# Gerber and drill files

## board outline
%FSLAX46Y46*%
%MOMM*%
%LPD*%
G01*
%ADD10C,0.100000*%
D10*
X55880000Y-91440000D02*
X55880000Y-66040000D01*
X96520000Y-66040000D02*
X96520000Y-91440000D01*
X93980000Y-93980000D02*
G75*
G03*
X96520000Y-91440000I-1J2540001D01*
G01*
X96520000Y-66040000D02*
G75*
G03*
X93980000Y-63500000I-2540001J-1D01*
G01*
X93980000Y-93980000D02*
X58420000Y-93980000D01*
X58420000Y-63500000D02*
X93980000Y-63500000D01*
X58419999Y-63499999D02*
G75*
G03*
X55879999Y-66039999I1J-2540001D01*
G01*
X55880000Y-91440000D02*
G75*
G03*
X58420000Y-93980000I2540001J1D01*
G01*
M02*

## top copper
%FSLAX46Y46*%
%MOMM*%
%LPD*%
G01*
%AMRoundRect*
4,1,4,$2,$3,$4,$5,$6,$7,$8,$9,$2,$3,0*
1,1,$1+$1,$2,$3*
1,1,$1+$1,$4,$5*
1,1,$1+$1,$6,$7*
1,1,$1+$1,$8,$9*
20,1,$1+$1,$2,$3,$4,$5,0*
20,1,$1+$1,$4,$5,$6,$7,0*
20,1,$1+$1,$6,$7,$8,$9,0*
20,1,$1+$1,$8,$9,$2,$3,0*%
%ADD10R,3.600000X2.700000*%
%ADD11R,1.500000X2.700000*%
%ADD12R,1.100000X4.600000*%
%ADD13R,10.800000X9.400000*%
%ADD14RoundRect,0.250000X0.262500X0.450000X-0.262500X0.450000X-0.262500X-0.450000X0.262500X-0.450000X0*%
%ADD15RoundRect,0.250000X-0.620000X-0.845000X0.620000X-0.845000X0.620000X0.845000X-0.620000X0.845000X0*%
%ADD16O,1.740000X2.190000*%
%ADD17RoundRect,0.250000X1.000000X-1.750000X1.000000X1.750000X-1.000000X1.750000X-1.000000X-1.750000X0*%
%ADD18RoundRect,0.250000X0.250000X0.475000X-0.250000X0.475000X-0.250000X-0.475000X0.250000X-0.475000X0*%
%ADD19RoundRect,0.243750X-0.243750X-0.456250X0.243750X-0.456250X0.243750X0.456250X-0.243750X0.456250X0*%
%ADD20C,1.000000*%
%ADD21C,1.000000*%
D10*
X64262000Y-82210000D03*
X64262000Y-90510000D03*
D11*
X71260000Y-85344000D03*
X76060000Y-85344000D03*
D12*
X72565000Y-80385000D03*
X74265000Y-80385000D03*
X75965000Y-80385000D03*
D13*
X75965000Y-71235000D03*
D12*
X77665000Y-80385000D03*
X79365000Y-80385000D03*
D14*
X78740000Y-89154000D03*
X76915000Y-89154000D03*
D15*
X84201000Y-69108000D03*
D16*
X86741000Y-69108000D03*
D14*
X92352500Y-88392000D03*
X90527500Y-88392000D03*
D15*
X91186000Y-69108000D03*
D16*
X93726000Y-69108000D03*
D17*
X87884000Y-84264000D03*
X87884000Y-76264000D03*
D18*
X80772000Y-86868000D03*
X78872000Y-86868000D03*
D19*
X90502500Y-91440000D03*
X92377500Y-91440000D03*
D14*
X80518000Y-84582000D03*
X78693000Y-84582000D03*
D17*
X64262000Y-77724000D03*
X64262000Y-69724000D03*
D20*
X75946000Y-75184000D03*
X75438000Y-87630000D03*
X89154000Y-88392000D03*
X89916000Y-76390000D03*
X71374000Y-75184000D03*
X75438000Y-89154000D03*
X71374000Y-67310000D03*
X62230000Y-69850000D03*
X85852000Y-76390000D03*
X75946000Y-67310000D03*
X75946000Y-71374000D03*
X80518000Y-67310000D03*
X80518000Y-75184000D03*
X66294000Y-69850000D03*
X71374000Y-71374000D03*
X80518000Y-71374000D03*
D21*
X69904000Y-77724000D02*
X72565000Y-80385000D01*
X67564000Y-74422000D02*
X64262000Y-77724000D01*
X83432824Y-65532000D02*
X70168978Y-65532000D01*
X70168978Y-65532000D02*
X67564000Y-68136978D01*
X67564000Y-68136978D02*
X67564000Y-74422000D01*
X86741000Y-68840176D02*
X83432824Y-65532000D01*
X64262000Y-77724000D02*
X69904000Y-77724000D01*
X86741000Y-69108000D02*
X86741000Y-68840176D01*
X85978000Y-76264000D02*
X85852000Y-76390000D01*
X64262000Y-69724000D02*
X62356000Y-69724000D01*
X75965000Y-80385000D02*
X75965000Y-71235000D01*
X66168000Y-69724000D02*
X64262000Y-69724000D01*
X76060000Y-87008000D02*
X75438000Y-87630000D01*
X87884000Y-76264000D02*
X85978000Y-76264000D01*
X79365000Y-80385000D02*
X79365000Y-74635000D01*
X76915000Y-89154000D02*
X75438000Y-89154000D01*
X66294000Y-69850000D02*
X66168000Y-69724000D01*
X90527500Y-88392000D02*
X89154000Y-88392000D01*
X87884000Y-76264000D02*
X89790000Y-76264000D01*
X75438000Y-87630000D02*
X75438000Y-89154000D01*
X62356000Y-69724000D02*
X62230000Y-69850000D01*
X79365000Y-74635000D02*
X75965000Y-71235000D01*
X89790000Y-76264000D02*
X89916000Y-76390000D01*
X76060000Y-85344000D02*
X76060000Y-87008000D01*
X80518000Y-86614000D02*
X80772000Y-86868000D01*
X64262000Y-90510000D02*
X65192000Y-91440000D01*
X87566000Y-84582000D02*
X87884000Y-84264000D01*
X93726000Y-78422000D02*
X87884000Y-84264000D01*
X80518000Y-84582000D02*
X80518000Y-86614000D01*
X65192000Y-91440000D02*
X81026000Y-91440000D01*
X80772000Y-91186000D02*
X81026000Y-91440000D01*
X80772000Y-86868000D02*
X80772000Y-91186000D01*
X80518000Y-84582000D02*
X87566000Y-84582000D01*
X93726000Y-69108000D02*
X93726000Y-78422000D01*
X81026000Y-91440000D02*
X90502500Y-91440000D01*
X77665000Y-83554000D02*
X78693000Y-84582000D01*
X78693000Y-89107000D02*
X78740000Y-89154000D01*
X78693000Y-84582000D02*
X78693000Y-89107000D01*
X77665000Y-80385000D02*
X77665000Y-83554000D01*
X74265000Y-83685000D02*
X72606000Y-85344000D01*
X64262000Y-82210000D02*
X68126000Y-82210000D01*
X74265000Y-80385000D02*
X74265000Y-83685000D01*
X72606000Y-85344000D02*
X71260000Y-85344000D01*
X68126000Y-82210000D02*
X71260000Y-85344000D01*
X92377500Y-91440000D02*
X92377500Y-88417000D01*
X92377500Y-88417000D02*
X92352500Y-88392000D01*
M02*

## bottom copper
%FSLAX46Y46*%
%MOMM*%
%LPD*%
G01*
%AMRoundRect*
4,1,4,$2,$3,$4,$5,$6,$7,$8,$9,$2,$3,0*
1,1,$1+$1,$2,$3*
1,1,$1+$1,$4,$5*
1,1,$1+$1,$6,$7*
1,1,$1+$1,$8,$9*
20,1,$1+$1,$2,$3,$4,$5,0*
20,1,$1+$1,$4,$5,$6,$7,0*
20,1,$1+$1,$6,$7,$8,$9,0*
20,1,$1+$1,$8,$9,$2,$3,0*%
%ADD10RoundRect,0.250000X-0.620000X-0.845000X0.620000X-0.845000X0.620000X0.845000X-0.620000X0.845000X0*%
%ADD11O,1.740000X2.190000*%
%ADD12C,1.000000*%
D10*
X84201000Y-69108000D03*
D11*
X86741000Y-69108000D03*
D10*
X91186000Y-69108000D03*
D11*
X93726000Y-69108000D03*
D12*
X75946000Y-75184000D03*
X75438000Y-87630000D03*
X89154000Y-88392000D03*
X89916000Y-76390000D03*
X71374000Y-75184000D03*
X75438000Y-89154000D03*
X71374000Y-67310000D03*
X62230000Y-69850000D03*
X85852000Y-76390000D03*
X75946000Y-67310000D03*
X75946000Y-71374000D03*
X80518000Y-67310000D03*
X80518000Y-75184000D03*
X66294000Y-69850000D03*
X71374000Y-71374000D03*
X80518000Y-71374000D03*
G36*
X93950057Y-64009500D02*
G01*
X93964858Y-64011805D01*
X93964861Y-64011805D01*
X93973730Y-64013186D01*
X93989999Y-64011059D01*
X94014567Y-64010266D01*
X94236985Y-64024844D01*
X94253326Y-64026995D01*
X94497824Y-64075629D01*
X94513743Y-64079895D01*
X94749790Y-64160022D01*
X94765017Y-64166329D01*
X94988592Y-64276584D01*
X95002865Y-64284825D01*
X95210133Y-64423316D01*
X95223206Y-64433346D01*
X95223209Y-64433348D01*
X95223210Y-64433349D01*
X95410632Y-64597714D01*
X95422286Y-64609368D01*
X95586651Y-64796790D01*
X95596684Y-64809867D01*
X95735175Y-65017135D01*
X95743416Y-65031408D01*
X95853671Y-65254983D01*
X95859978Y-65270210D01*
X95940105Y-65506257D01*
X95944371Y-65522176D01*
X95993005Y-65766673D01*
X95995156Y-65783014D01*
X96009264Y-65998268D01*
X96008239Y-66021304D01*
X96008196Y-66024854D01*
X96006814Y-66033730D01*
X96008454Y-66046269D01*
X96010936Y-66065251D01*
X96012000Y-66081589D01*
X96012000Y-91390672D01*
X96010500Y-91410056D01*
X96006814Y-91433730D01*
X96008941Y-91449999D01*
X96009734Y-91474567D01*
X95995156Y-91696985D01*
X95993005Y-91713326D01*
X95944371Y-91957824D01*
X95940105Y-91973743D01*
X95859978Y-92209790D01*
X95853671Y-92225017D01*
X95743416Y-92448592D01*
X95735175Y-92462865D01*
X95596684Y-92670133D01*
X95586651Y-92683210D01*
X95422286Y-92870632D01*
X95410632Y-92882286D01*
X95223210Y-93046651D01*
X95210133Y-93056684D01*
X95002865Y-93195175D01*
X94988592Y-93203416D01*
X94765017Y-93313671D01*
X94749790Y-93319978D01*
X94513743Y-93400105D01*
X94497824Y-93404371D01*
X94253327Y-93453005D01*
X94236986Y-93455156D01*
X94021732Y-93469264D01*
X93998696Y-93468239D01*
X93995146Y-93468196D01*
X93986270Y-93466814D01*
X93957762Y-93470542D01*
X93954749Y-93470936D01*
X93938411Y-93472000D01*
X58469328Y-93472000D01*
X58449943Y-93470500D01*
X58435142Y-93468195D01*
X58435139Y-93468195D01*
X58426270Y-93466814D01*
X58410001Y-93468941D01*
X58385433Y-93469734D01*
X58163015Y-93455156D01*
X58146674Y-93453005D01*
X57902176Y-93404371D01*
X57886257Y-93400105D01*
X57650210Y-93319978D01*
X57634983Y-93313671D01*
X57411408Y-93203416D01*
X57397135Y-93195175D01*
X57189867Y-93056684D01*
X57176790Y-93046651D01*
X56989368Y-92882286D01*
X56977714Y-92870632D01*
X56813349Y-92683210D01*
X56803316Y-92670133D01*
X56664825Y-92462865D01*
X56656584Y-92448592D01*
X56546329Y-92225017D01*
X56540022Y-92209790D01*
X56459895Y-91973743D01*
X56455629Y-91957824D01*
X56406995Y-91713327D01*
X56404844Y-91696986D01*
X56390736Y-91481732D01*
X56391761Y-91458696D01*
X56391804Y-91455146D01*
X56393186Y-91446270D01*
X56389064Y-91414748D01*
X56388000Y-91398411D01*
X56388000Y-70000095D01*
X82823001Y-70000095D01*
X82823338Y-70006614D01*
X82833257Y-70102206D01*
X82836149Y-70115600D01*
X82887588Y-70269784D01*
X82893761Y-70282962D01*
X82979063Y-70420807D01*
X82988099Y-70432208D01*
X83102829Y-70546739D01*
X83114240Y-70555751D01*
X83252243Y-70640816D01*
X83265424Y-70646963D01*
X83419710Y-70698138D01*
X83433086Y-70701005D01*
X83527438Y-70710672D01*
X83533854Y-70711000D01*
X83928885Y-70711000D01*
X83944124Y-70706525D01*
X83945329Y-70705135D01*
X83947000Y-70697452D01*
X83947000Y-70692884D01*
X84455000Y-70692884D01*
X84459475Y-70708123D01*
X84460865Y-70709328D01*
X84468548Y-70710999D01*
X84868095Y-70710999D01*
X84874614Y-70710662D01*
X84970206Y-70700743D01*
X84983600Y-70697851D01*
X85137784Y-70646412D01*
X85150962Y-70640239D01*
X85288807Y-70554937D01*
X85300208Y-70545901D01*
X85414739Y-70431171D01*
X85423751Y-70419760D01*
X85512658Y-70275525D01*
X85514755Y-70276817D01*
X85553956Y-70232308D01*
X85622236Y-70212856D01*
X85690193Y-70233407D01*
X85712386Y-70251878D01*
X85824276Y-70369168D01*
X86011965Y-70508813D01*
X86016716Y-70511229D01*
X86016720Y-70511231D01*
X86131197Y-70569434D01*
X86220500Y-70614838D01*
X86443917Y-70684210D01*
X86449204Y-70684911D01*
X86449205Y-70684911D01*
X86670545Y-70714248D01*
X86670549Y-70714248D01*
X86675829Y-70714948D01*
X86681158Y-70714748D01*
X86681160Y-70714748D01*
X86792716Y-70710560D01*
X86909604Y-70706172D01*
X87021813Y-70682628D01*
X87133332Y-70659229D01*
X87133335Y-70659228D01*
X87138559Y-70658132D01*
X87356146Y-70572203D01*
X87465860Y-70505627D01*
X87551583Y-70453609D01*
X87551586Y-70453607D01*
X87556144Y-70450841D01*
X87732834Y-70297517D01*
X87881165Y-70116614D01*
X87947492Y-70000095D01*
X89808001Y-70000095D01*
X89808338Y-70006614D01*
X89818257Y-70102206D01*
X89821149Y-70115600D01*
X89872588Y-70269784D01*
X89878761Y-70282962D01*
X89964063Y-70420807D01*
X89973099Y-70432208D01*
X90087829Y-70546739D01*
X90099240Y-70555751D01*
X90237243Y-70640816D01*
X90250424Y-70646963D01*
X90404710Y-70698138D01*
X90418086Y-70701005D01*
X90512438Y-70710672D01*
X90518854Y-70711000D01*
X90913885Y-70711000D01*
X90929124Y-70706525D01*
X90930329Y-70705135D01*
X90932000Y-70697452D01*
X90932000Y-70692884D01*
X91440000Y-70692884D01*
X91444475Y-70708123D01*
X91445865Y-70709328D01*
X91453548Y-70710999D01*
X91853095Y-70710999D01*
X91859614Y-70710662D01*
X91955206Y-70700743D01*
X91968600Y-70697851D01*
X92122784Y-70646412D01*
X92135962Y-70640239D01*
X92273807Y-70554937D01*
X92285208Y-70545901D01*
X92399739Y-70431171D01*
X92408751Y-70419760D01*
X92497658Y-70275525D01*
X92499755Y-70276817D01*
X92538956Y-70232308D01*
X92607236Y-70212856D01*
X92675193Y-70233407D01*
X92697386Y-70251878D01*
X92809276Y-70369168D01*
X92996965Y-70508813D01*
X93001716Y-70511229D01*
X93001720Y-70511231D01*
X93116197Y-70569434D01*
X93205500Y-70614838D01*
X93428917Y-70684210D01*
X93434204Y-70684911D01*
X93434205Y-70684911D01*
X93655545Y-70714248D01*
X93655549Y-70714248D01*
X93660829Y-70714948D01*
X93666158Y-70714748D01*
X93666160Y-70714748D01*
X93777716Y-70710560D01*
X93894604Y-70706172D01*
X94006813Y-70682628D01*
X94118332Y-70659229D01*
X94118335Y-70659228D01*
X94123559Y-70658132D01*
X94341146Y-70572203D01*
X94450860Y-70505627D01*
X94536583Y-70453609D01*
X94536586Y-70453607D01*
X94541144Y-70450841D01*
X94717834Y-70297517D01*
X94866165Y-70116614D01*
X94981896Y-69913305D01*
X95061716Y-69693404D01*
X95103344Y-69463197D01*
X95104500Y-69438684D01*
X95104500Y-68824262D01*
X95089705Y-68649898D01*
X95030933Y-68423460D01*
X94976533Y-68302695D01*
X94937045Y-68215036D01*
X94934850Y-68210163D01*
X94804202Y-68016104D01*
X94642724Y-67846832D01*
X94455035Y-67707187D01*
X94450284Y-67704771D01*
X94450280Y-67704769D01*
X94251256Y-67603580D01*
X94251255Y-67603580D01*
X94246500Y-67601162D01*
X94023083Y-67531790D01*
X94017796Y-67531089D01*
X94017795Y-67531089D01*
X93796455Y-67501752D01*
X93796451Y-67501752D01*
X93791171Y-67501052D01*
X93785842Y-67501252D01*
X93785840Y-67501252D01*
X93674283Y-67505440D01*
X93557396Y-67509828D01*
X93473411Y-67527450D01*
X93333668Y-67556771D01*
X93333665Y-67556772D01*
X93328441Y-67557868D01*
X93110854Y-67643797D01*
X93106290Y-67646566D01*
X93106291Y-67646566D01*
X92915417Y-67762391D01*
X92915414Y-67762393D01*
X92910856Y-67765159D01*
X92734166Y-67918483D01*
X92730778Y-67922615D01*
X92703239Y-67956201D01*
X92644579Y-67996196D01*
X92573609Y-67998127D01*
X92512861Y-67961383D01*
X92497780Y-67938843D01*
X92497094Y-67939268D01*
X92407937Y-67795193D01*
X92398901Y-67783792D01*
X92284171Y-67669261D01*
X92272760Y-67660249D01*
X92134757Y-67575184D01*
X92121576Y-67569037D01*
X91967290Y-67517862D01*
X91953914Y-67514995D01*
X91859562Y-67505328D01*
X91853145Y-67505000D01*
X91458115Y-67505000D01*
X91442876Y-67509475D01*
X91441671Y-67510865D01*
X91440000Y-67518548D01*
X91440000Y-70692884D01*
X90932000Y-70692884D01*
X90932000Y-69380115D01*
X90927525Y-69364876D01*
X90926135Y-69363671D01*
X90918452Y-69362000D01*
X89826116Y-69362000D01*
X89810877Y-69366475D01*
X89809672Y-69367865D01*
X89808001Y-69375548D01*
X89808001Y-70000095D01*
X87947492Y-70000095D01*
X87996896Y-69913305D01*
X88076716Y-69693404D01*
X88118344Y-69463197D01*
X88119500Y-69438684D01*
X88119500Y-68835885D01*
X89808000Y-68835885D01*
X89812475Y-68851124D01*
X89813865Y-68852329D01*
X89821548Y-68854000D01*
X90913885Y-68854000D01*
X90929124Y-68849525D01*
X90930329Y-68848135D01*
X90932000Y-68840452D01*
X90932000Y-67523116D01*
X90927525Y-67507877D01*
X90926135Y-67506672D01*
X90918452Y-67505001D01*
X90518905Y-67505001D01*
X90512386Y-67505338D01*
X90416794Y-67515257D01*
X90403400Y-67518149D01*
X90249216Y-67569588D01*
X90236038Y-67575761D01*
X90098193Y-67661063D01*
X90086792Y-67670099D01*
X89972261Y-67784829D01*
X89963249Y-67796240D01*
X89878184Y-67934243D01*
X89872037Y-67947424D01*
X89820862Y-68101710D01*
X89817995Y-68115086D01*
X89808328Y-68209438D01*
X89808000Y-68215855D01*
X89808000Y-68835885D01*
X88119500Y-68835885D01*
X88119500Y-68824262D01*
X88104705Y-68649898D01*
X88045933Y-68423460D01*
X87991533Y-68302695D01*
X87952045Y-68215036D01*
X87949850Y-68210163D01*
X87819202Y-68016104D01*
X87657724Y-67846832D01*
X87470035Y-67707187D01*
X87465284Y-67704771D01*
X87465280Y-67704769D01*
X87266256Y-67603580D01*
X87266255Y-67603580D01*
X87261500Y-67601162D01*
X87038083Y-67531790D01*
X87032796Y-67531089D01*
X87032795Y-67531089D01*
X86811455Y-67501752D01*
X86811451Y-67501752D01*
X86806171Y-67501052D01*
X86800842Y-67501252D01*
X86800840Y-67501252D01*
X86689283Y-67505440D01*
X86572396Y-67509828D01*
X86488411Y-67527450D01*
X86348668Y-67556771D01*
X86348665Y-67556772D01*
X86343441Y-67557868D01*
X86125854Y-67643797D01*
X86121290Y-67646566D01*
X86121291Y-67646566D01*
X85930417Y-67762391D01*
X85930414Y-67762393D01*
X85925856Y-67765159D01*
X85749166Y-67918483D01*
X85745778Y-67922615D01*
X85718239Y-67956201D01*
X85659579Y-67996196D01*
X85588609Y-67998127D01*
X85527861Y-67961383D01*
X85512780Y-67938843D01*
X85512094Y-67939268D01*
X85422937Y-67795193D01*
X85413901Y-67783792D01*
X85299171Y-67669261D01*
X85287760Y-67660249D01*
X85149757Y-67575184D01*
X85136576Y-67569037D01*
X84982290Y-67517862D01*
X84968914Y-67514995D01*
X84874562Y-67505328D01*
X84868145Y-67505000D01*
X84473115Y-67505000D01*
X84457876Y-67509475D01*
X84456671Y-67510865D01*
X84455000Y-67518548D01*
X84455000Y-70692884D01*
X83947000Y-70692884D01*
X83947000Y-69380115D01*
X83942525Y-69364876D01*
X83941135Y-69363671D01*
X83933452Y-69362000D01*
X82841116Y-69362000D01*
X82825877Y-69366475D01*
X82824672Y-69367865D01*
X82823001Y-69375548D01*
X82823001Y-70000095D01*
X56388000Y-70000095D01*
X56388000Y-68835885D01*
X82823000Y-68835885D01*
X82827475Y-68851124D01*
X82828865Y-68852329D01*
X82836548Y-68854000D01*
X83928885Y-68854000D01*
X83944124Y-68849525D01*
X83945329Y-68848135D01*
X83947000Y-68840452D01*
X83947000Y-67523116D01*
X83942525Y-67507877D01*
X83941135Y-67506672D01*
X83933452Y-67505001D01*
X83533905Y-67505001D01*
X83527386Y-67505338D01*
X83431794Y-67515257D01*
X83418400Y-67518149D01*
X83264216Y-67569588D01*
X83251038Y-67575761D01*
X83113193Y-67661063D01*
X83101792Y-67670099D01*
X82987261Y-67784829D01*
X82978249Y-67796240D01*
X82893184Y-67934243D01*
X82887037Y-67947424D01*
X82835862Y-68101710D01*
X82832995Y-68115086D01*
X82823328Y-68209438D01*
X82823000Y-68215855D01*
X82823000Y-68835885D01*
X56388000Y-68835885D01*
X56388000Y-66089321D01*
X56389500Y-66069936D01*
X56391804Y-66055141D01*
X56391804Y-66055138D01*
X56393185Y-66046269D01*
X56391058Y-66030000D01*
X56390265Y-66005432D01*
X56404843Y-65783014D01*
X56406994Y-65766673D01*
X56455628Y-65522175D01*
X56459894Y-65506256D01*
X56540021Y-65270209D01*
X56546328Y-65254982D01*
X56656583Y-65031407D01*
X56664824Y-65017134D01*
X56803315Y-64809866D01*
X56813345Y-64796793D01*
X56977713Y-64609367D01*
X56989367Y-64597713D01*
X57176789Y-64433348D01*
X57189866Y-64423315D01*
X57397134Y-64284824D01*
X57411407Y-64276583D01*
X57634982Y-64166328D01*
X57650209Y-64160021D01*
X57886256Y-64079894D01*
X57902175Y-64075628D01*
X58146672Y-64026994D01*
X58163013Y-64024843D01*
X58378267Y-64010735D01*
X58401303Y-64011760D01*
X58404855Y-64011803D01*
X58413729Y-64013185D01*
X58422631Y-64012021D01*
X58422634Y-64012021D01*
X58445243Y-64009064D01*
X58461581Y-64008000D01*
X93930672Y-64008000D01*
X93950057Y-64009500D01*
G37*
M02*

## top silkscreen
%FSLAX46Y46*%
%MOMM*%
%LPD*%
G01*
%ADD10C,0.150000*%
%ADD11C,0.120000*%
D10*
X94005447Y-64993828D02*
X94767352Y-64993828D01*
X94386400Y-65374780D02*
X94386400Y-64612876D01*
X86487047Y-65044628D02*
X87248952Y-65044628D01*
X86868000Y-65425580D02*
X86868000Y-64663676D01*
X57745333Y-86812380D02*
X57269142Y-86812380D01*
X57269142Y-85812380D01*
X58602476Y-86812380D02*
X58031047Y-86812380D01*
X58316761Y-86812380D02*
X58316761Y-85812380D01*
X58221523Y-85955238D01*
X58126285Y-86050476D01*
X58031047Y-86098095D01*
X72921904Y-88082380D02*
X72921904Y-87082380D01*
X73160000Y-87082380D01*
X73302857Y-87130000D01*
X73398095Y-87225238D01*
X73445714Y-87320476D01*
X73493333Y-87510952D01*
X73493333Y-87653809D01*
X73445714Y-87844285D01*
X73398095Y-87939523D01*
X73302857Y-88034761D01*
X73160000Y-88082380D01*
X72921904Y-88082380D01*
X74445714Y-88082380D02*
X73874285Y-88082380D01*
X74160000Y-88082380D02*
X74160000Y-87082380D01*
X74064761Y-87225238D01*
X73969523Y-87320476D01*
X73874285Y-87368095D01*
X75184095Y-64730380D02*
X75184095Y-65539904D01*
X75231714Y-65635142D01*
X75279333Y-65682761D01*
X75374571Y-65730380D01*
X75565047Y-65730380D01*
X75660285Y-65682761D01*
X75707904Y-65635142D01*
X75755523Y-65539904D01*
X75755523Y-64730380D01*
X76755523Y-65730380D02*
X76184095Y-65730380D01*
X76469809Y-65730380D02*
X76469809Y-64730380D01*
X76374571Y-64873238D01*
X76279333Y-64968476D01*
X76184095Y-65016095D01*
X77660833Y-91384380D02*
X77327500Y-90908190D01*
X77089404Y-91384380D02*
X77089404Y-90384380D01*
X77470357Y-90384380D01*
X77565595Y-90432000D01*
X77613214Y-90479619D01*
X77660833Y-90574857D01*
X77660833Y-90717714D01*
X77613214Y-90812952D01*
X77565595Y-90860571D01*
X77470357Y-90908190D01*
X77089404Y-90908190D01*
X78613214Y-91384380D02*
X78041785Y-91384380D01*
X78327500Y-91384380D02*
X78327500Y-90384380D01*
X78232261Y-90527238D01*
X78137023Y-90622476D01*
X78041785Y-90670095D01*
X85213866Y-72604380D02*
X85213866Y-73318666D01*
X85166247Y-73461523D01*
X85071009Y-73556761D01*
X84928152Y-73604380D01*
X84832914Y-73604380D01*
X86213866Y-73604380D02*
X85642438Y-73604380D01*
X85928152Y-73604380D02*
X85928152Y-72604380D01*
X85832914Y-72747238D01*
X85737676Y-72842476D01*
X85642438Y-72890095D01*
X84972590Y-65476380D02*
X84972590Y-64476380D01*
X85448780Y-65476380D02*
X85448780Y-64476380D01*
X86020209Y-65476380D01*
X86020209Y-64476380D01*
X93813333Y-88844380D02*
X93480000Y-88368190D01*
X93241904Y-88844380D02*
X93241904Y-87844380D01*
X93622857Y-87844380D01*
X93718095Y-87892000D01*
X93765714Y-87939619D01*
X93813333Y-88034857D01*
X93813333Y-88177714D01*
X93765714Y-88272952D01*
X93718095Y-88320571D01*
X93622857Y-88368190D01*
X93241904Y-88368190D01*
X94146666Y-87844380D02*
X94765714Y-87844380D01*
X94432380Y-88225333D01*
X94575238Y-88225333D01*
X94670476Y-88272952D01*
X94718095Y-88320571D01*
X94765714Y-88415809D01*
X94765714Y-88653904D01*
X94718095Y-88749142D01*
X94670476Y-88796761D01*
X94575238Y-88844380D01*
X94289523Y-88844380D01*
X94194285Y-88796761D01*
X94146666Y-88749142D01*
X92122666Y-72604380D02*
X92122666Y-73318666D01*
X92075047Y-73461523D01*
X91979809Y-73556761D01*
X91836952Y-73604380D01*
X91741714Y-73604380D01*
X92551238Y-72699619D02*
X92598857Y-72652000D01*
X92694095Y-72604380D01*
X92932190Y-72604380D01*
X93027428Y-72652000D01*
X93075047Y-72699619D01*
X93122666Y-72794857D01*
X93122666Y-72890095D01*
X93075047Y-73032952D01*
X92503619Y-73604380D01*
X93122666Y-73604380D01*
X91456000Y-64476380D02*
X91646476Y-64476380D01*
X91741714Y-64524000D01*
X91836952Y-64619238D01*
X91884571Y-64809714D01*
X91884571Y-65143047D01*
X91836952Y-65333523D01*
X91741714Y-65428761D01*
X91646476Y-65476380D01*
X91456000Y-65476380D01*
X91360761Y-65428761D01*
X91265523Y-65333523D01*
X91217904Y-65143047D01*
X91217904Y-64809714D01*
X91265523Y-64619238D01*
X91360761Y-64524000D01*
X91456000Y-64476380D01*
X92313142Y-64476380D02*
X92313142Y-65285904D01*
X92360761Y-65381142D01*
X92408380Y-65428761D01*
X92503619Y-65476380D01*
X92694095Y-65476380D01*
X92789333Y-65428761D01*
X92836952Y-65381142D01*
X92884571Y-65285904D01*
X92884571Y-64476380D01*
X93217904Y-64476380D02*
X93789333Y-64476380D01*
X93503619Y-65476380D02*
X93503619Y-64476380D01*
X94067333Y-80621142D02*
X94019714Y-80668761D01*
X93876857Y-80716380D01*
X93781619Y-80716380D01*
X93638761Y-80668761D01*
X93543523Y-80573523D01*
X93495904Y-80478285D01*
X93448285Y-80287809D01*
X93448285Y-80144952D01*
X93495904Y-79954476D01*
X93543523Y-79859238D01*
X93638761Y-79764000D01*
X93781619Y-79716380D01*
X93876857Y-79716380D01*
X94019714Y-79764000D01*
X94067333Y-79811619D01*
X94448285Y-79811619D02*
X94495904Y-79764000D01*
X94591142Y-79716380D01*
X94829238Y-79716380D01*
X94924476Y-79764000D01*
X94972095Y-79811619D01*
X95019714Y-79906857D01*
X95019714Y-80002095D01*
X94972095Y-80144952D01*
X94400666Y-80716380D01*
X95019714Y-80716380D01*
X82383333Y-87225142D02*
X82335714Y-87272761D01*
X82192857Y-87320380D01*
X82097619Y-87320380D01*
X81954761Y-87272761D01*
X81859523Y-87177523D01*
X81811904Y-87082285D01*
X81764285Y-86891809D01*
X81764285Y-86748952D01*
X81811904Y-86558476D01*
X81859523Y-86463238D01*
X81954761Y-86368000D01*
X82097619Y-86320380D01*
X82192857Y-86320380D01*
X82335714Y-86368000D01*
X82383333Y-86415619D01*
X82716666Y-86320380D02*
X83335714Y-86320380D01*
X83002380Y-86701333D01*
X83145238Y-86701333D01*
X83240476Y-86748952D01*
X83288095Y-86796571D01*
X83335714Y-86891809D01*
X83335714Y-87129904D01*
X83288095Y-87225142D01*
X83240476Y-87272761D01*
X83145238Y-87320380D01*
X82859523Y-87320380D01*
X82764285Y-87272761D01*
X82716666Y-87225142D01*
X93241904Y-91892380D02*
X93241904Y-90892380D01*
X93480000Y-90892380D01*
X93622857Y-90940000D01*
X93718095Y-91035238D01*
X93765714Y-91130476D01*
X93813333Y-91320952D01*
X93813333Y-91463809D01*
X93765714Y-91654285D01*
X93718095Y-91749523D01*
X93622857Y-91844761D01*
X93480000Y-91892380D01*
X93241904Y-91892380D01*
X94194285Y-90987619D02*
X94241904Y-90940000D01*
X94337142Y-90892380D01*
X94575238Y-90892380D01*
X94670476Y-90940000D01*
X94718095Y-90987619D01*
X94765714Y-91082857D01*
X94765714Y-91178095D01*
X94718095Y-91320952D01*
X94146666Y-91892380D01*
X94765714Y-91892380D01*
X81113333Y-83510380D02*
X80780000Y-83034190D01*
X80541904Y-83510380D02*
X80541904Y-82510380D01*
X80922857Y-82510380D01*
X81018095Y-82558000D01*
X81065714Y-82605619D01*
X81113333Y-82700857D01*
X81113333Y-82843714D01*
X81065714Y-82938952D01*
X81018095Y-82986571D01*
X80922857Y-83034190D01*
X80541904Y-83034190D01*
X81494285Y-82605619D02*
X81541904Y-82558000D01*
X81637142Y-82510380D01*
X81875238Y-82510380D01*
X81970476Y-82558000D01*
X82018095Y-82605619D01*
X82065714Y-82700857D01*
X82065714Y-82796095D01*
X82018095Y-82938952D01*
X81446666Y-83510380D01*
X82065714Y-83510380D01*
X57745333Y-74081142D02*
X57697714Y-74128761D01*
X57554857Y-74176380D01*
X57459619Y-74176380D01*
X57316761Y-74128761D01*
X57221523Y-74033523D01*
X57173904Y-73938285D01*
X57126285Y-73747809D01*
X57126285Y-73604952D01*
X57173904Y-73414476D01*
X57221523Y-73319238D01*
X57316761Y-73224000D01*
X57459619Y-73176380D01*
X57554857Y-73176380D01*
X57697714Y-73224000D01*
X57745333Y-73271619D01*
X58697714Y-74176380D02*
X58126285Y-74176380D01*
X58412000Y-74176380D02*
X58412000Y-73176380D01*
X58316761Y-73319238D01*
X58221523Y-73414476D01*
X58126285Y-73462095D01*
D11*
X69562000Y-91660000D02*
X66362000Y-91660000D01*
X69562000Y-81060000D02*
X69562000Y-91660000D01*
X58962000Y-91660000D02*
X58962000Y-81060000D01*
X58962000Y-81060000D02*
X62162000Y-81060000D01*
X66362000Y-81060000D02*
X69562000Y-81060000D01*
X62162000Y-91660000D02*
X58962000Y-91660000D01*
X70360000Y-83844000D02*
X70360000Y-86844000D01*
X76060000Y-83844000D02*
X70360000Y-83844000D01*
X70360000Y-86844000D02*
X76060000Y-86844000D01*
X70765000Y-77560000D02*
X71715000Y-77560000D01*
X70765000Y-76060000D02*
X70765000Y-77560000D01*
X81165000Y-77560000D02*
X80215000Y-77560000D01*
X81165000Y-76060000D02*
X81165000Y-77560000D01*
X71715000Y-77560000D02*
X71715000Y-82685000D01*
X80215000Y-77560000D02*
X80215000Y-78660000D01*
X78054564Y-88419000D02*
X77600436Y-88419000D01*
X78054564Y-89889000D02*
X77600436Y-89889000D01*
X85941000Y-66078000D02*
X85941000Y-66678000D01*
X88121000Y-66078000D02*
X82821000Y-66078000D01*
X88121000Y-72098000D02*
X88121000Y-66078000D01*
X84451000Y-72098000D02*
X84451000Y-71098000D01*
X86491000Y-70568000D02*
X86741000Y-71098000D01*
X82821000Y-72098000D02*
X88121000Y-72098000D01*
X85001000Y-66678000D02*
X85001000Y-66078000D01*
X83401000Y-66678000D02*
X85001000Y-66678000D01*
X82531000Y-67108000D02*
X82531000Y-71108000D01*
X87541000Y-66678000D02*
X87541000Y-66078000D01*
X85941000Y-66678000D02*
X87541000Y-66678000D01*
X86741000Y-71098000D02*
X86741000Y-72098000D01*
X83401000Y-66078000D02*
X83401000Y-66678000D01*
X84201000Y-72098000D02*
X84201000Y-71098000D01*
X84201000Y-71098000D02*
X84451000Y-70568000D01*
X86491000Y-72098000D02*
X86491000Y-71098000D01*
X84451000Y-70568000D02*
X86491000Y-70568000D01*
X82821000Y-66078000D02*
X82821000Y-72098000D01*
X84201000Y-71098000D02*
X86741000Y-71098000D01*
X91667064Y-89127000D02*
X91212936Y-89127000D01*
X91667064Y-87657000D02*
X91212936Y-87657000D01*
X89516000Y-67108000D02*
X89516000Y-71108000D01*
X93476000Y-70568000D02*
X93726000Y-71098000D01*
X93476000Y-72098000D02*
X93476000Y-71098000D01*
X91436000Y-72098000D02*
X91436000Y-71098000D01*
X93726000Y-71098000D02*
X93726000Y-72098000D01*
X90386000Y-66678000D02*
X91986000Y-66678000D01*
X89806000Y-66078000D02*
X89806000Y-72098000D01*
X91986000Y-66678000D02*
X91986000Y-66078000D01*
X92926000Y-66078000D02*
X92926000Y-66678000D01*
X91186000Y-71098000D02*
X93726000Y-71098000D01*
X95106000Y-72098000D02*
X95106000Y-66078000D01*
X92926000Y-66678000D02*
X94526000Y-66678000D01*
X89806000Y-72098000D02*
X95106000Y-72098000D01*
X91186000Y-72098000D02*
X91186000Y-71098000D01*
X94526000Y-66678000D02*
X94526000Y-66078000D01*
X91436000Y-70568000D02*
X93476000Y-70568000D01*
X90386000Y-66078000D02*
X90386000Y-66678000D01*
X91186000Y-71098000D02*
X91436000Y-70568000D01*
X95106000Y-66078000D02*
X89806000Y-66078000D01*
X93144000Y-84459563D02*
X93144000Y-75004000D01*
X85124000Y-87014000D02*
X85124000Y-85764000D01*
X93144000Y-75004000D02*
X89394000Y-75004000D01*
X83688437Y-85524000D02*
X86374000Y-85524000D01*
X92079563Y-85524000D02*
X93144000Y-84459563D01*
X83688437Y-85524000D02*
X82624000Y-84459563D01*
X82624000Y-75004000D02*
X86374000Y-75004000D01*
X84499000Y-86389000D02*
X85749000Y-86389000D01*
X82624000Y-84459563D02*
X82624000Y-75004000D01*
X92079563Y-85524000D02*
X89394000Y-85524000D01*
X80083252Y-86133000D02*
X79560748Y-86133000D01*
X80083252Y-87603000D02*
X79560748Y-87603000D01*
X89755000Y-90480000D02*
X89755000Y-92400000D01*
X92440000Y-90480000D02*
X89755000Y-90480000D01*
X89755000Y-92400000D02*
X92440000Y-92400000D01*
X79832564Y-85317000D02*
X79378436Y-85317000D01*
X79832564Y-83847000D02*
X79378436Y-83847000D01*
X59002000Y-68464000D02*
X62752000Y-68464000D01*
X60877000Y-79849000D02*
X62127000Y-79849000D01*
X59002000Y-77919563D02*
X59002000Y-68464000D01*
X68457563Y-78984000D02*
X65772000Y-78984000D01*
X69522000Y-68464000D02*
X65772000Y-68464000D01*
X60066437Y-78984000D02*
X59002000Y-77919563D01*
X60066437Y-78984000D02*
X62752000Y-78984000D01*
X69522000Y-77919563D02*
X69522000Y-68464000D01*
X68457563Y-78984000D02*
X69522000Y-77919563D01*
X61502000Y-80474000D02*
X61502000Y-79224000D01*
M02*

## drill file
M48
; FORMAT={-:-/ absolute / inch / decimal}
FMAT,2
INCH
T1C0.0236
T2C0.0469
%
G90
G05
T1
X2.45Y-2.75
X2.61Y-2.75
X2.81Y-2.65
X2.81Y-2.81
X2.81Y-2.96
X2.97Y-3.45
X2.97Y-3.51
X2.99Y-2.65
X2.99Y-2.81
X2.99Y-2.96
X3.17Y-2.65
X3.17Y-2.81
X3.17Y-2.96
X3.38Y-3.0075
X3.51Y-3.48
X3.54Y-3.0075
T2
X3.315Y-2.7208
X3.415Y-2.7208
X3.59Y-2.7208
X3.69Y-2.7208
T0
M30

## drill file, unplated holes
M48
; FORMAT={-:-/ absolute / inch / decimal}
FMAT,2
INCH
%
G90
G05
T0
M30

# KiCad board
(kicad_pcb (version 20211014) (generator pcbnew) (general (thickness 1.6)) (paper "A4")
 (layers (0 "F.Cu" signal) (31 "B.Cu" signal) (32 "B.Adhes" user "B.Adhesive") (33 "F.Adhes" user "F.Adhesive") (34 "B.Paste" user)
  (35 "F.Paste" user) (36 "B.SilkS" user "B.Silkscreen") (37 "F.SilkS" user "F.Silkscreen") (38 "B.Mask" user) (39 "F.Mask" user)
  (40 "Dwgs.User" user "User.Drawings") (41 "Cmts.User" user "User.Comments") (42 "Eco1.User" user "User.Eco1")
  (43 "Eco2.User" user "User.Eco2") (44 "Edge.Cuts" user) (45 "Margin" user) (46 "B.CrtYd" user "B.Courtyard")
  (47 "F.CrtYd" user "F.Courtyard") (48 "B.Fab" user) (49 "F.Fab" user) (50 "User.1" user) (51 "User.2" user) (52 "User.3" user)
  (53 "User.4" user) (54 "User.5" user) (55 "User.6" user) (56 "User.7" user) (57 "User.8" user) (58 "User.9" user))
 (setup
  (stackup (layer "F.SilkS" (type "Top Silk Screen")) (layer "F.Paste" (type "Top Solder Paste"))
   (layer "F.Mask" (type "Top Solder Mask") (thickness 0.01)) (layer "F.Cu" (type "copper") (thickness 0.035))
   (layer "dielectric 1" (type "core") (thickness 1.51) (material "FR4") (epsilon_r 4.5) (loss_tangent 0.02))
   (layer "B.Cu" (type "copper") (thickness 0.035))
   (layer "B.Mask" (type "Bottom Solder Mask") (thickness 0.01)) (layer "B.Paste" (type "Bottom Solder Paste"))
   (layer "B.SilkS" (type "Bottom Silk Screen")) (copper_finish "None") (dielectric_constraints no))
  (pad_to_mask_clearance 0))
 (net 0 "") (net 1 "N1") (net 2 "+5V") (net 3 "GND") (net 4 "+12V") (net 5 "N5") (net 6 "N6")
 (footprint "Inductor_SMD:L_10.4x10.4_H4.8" (layer "F.Cu") (at 64.262 86.36 -90)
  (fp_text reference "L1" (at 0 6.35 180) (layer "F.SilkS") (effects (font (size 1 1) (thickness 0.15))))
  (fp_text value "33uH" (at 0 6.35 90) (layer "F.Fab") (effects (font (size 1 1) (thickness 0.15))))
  (fp_line (start 5.3 -5.3) (end 5.3 -2.1) (layer "F.SilkS") (width 0.12))
  (fp_line (start -5.3 -5.3) (end 5.3 -5.3) (layer "F.SilkS") (width 0.12))
  (fp_line (start 5.3 5.3) (end -5.3 5.3) (layer "F.SilkS") (width 0.12))
  (fp_line (start -5.3 5.3) (end -5.3 2.1) (layer "F.SilkS") (width 0.12))
  (fp_line (start -5.3 -2.1) (end -5.3 -5.3) (layer "F.SilkS") (width 0.12))
  (fp_line (start 5.3 2.1) (end 5.3 5.3) (layer "F.SilkS") (width 0.12))
  (pad "1" smd rect locked (at -4.15 0 270) (size 2.7 3.6) (layers "F.Cu" "F.Paste" "F.Mask") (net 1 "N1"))
  (pad "2" smd rect locked (at 4.15 0 270) (size 2.7 3.6) (layers "F.Cu" "F.Paste" "F.Mask") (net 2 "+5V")))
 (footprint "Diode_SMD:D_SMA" (layer "F.Cu") (at 73.66 85.344)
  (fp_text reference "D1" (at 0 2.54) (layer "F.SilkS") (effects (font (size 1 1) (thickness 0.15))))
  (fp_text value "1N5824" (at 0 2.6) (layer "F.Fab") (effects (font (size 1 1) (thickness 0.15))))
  (fp_line (start -3.4 -1.65) (end 2 -1.65) (layer "F.SilkS") (width 0.12))
  (fp_line (start -3.4 -1.65) (end -3.4 1.65) (layer "F.SilkS") (width 0.12))
  (fp_line (start -3.4 1.65) (end 2 1.65) (layer "F.SilkS") (width 0.12))
  (pad "1" smd rect locked (at -2 0) (size 2.5 1.8) (layers "F.Cu" "F.Paste" "F.Mask") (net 1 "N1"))
  (pad "2" smd rect locked (at 2 0) (size 2.5 1.8) (layers "F.Cu" "F.Paste" "F.Mask") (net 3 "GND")))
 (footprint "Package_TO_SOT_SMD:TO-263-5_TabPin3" (layer "F.Cu") (at 75.965 74.61 90)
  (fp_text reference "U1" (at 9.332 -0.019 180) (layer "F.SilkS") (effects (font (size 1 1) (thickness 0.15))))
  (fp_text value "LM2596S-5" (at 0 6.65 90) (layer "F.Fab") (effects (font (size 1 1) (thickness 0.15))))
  (fp_line (start -2.95 -5.2) (end -2.95 -4.25) (layer "F.SilkS") (width 0.12))
  (fp_line (start -1.45 -5.2) (end -2.95 -5.2) (layer "F.SilkS") (width 0.12))
  (fp_line (start -2.95 5.2) (end -2.95 4.25) (layer "F.SilkS") (width 0.12))
  (fp_line (start -1.45 5.2) (end -2.95 5.2) (layer "F.SilkS") (width 0.12))
  (fp_line (start -2.95 -4.25) (end -8.075 -4.25) (layer "F.SilkS") (width 0.12))
  (fp_line (start -2.95 4.25) (end -4.05 4.25) (layer "F.SilkS") (width 0.12))
  (pad "" smd rect locked (at 5.8 -2.775 90) (size 4.55 5.25) (layers "F.Paste"))
  (pad "" smd rect locked (at 5.8 2.775 90) (size 4.55 5.25) (layers "F.Paste"))
  (pad "" smd rect locked (at 0.95 2.775 90) (size 4.55 5.25) (layers "F.Paste"))
  (pad "" smd rect locked (at 0.95 -2.775 90) (size 4.55 5.25) (layers "F.Paste"))
  (pad "1" smd rect locked (at -5.775 -3.4 90) (size 4.6 1.1) (layers "F.Cu" "F.Paste" "F.Mask") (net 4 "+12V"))
  (pad "2" smd rect locked (at -5.775 -1.7 90) (size 4.6 1.1) (layers "F.Cu" "F.Paste" "F.Mask") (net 1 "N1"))
  (pad "3" smd rect locked (at -5.775 0 90) (size 4.6 1.1) (layers "F.Cu" "F.Paste" "F.Mask") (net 3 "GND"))
  (pad "3" smd rect locked (at 3.375 0 90) (size 9.4 10.8) (layers "F.Cu" "F.Mask") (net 3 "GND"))
  (pad "4" smd rect locked (at -5.775 1.7 90) (size 4.6 1.1) (layers "F.Cu" "F.Paste" "F.Mask") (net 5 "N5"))
  (pad "5" smd rect locked (at -5.775 3.4 90) (size 4.6 1.1) (layers "F.Cu" "F.Paste" "F.Mask") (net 3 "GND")))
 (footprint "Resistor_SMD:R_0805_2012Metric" (layer "F.Cu") (at 77.8275 89.154 180)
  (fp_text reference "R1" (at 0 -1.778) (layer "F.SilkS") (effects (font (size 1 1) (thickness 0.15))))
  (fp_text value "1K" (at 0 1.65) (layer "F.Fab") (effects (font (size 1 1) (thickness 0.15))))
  (fp_line (start -0.227064 0.735) (end 0.227064 0.735) (layer "F.SilkS") (width 0.12))
  (fp_line (start -0.227064 -0.735) (end 0.227064 -0.735) (layer "F.SilkS") (width 0.12))
  (pad "1" smd roundrect locked (at -0.9125 0 180) (size 1.025 1.4) (layers "F.Cu" "F.Paste" "F.Mask") (roundrect_rratio 0.243902439)
   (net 5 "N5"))
  (pad "2" smd roundrect locked (at 0.9125 0 180) (size 1.025 1.4) (layers "F.Cu" "F.Paste" "F.Mask") (roundrect_rratio 0.243902439)
   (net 3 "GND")))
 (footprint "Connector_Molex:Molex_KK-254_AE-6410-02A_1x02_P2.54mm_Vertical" (layer "F.Cu") (at 84.201 69.108)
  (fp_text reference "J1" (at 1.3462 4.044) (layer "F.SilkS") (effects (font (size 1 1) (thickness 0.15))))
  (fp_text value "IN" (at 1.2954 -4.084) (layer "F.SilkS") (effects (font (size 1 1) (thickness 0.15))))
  (fp_line (start 1.74 -3.03) (end 1.74 -2.43) (layer "F.SilkS") (width 0.12))
  (fp_line (start 3.92 -3.03) (end -1.38 -3.03) (layer "F.SilkS") (width 0.12))
  (fp_line (start 3.92 2.99) (end 3.92 -3.03) (layer "F.SilkS") (width 0.12))
  (fp_line (start 0.25 2.99) (end 0.25 1.99) (layer "F.SilkS") (width 0.12))
  (fp_line (start 2.29 1.46) (end 2.54 1.99) (layer "F.SilkS") (width 0.12))
  (fp_line (start -1.38 2.99) (end 3.92 2.99) (layer "F.SilkS") (width 0.12))
  (fp_line (start 0.8 -2.43) (end 0.8 -3.03) (layer "F.SilkS") (width 0.12))
  (fp_line (start -0.8 -2.43) (end 0.8 -2.43) (layer "F.SilkS") (width 0.12))
  (fp_line (start -1.67 -2) (end -1.67 2) (layer "F.SilkS") (width 0.12))
  (fp_line (start 3.34 -2.43) (end 3.34 -3.03) (layer "F.SilkS") (width 0.12))
  (fp_line (start 1.74 -2.43) (end 3.34 -2.43) (layer "F.SilkS") (width 0.12))
  (fp_line (start 2.54 1.99) (end 2.54 2.99) (layer "F.SilkS") (width 0.12))
  (fp_line (start -0.8 -3.03) (end -0.8 -2.43) (layer "F.SilkS") (width 0.12))
  (fp_line (start 0 2.99) (end 0 1.99) (layer "F.SilkS") (width 0.12))
  (fp_line (start 0 1.99) (end 0.25 1.46) (layer "F.SilkS") (width 0.12))
  (fp_line (start 2.29 2.99) (end 2.29 1.99) (layer "F.SilkS") (width 0.12))
  (fp_line (start 0.25 1.46) (end 2.29 1.46) (layer "F.SilkS") (width 0.12))
  (fp_line (start -1.38 -3.03) (end -1.38 2.99) (layer "F.SilkS") (width 0.12))
  (fp_line (start 0 1.99) (end 2.54 1.99) (layer "F.SilkS") (width 0.12))
  (pad "1" thru_hole roundrect locked (at 0 0) (size 1.74 2.19) (drill 1.19) (layers *.Cu *.Mask) (roundrect_rratio 0.1436781609)
   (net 3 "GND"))
  (pad "2" thru_hole oval locked (at 2.54 0) (size 1.74 2.19) (drill 1.19) (layers *.Cu *.Mask) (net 4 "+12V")))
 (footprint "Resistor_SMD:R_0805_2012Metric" (layer "F.Cu") (at 91.44 88.392 180)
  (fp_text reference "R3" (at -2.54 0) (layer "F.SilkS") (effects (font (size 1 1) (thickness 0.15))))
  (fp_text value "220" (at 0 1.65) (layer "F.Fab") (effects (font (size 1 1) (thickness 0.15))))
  (fp_line (start -0.227064 -0.735) (end 0.227064 -0.735) (layer "F.SilkS") (width 0.12))
  (fp_line (start -0.227064 0.735) (end 0.227064 0.735) (layer "F.SilkS") (width 0.12))
  (pad "1" smd roundrect locked (at -0.9125 0 180) (size 1.025 1.4) (layers "F.Cu" "F.Paste" "F.Mask") (roundrect_rratio 0.243902439)
   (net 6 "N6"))
  (pad "2" smd roundrect locked (at 0.9125 0 180) (size 1.025 1.4) (layers "F.Cu" "F.Paste" "F.Mask") (roundrect_rratio 0.243902439)
   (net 3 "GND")))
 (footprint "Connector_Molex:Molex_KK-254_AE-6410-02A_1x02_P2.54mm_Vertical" (layer "F.Cu") (at 91.186 69.108)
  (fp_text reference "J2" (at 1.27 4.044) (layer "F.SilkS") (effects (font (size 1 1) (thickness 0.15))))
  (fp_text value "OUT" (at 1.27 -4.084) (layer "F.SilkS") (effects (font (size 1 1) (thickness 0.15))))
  (fp_line (start -1.67 -2) (end -1.67 2) (layer "F.SilkS") (width 0.12))
  (fp_line (start 2.29 1.46) (end 2.54 1.99) (layer "F.SilkS") (width 0.12))
  (fp_line (start 2.29 2.99) (end 2.29 1.99) (layer "F.SilkS") (width 0.12))
  (fp_line (start 0.25 2.99) (end 0.25 1.99) (layer "F.SilkS") (width 0.12))
  (fp_line (start 2.54 1.99) (end 2.54 2.99) (layer "F.SilkS") (width 0.12))
  (fp_line (start -0.8 -2.43) (end 0.8 -2.43) (layer "F.SilkS") (width 0.12))
  (fp_line (start -1.38 -3.03) (end -1.38 2.99) (layer "F.SilkS") (width 0.12))
  (fp_line (start 0.8 -2.43) (end 0.8 -3.03) (layer "F.SilkS") (width 0.12))
  (fp_line (start 1.74 -3.03) (end 1.74 -2.43) (layer "F.SilkS") (width 0.12))
  (fp_line (start 0 1.99) (end 2.54 1.99) (layer "F.SilkS") (width 0.12))
  (fp_line (start 3.92 2.99) (end 3.92 -3.03) (layer "F.SilkS") (width 0.12))
  (fp_line (start 1.74 -2.43) (end 3.34 -2.43) (layer "F.SilkS") (width 0.12))
  (fp_line (start -1.38 2.99) (end 3.92 2.99) (layer "F.SilkS") (width 0.12))
  (fp_line (start 0 2.99) (end 0 1.99) (layer "F.SilkS") (width 0.12))
  (fp_line (start 3.34 -2.43) (end 3.34 -3.03) (layer "F.SilkS") (width 0.12))
  (fp_line (start 0.25 1.46) (end 2.29 1.46) (layer "F.SilkS") (width 0.12))
  (fp_line (start -0.8 -3.03) (end -0.8 -2.43) (layer "F.SilkS") (width 0.12))
  (fp_line (start 0 1.99) (end 0.25 1.46) (layer "F.SilkS") (width 0.12))
  (fp_line (start 3.92 -3.03) (end -1.38 -3.03) (layer "F.SilkS") (width 0.12))
  (pad "1" thru_hole roundrect locked (at 0 0) (size 1.74 2.19) (drill 1.19) (layers *.Cu *.Mask) (roundrect_rratio 0.1436781609)
   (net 3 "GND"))
  (pad "2" thru_hole oval locked (at 2.54 0) (size 1.74 2.19) (drill 1.19) (layers *.Cu *.Mask) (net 2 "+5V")))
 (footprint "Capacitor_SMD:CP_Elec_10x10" (layer "F.Cu") (at 87.884 80.264 90)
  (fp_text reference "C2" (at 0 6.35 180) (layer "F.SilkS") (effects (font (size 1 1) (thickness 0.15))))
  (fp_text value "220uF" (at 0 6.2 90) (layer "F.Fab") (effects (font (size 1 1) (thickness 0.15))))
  (fp_line (start -4.195563 5.26) (end 5.26 5.26) (layer "F.SilkS") (width 0.12))
  (fp_line (start -6.75 -2.76) (end -5.5 -2.76) (layer "F.SilkS") (width 0.12))
  (fp_line (start 5.26 5.26) (end 5.26 1.51) (layer "F.SilkS") (width 0.12))
  (fp_line (start -5.26 -4.195563) (end -5.26 -1.51) (layer "F.SilkS") (width 0.12))
  (fp_line (start -5.26 4.195563) (end -4.195563 5.26) (layer "F.SilkS") (width 0.12))
  (fp_line (start -5.26 -4.195563) (end -4.195563 -5.26) (layer "F.SilkS") (width 0.12))
  (fp_line (start 5.26 -5.26) (end 5.26 -1.51) (layer "F.SilkS") (width 0.12))
  (fp_line (start -6.125 -3.385) (end -6.125 -2.135) (layer "F.SilkS") (width 0.12))
  (fp_line (start -4.195563 -5.26) (end 5.26 -5.26) (layer "F.SilkS") (width 0.12))
  (fp_line (start -5.26 4.195563) (end -5.26 1.51) (layer "F.SilkS") (width 0.12))
  (pad "1" smd roundrect locked (at -4 0 90) (size 4 2.5) (layers "F.Cu" "F.Paste" "F.Mask") (roundrect_rratio 0.1) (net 2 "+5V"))
  (pad "2" smd roundrect locked (at 4 0 90) (size 4 2.5) (layers "F.Cu" "F.Paste" "F.Mask") (roundrect_rratio 0.1) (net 3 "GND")))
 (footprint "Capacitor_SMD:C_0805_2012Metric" (layer "F.Cu") (at 79.822 86.868 180)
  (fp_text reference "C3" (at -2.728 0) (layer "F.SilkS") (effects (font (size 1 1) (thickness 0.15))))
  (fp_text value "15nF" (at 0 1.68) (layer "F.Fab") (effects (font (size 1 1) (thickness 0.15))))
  (fp_line (start -0.261252 0.735) (end 0.261252 0.735) (layer "F.SilkS") (width 0.12))
  (fp_line (start -0.261252 -0.735) (end 0.261252 -0.735) (layer "F.SilkS") (width 0.12))
  (pad "1" smd roundrect locked (at -0.95 0 180) (size 1 1.45) (layers "F.Cu" "F.Paste" "F.Mask") (roundrect_rratio 0.25) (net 2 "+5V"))
  (pad "2" smd roundrect locked (at 0.95 0 180) (size 1 1.45) (layers "F.Cu" "F.Paste" "F.Mask") (roundrect_rratio 0.25) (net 5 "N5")))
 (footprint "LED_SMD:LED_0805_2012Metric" (layer "F.Cu") (at 91.44 91.44)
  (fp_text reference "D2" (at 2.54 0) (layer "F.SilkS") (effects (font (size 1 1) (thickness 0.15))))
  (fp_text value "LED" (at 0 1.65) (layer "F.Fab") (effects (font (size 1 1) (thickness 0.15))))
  (fp_line (start -1.685 -0.96) (end -1.685 0.96) (layer "F.SilkS") (width 0.12))
  (fp_line (start 1 -0.96) (end -1.685 -0.96) (layer "F.SilkS") (width 0.12))
  (fp_line (start -1.685 0.96) (end 1 0.96) (layer "F.SilkS") (width 0.12))
  (pad "1" smd roundrect locked (at -0.9375 0) (size 0.975 1.4) (layers "F.Cu" "F.Paste" "F.Mask") (roundrect_rratio 0.25) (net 2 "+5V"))
  (pad "2" smd roundrect locked (at 0.9375 0) (size 0.975 1.4) (layers "F.Cu" "F.Paste" "F.Mask") (roundrect_rratio 0.25) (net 6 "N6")))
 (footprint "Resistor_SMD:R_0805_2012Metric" (layer "F.Cu") (at 79.6055 84.582 180)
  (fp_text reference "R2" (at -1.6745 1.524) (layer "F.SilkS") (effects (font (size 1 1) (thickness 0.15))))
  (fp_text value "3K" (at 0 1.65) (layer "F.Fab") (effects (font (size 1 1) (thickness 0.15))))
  (fp_line (start -0.227064 -0.735) (end 0.227064 -0.735) (layer "F.SilkS") (width 0.12))
  (fp_line (start -0.227064 0.735) (end 0.227064 0.735) (layer "F.SilkS") (width 0.12))
  (pad "1" smd roundrect locked (at -0.9125 0 180) (size 1.025 1.4) (layers "F.Cu" "F.Paste" "F.Mask") (roundrect_rratio 0.243902439)
   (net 2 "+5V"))
  (pad "2" smd roundrect locked (at 0.9125 0 180) (size 1.025 1.4) (layers "F.Cu" "F.Paste" "F.Mask") (roundrect_rratio 0.243902439)
   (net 5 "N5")))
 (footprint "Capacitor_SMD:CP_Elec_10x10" (layer "F.Cu") (at 64.262 73.724 90)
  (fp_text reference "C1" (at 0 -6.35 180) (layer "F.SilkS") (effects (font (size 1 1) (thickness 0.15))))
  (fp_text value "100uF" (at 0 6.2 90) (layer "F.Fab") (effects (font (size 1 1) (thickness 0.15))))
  (fp_line (start 5.26 -5.26) (end 5.26 -1.51) (layer "F.SilkS") (width 0.12))
  (fp_line (start -6.125 -3.385) (end -6.125 -2.135) (layer "F.SilkS") (width 0.12))
  (fp_line (start -4.195563 -5.26) (end 5.26 -5.26) (layer "F.SilkS") (width 0.12))
  (fp_line (start -5.26 4.195563) (end -5.26 1.51) (layer "F.SilkS") (width 0.12))
  (fp_line (start 5.26 5.26) (end 5.26 1.51) (layer "F.SilkS") (width 0.12))
  (fp_line (start -5.26 -4.195563) (end -4.195563 -5.26) (layer "F.SilkS") (width 0.12))
  (fp_line (start -5.26 -4.195563) (end -5.26 -1.51) (layer "F.SilkS") (width 0.12))
  (fp_line (start -4.195563 5.26) (end 5.26 5.26) (layer "F.SilkS") (width 0.12))
  (fp_line (start -5.26 4.195563) (end -4.195563 5.26) (layer "F.SilkS") (width 0.12))
  (fp_line (start -6.75 -2.76) (end -5.5 -2.76) (layer "F.SilkS") (width 0.12))
  (pad "1" smd roundrect locked (at -4 0 90) (size 4 2.5) (layers "F.Cu" "F.Paste" "F.Mask") (roundrect_rratio 0.1) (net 4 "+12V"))
  (pad "2" smd roundrect locked (at 4 0 90) (size 4 2.5) (layers "F.Cu" "F.Paste" "F.Mask") (roundrect_rratio 0.1) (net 3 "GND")))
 (gr_line (start 55.88 91.44) (end 55.88 66.04) (layer "Edge.Cuts") (width 0.1))
 (gr_line (start 96.52 66.04) (end 96.52 91.44) (layer "Edge.Cuts") (width 0.1))
 (gr_arc (start 96.52 91.44) (mid 95.776051 93.236051) (end 93.98 93.98) (layer "Edge.Cuts") (width 0.1))
 (gr_arc (start 93.98 63.5) (mid 95.776051 64.243949) (end 96.52 66.04) (layer "Edge.Cuts") (width 0.1))
 (gr_line (start 93.98 93.98) (end 58.42 93.98) (layer "Edge.Cuts") (width 0.1))
 (gr_line (start 58.42 63.5) (end 93.98 63.5) (layer "Edge.Cuts") (width 0.1))
 (gr_arc (start 55.879999 66.039999) (mid 56.623948 64.243948) (end 58.419999 63.499999) (layer "Edge.Cuts") (width 0.1))
 (gr_arc (start 58.42 93.98) (mid 56.623949 93.236051) (end 55.88 91.44) (layer "Edge.Cuts") (width 0.1))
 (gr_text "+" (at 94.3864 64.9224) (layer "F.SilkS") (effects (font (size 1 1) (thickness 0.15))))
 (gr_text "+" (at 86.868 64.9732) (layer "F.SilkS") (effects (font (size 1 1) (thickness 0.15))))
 (segment (start 69.904 77.724) (end 72.565 80.385) (width 1) (layer "F.Cu") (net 4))
 (segment (start 67.564 74.422) (end 64.262 77.724) (width 1) (layer "F.Cu") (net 4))
 (segment (start 83.432824 65.532) (end 70.168978 65.532) (width 1) (layer "F.Cu") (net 4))
 (segment (start 70.168978 65.532) (end 67.564 68.136978) (width 1) (layer "F.Cu") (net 4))
 (segment (start 67.564 68.136978) (end 67.564 74.422) (width 1) (layer "F.Cu") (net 4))
 (segment (start 86.741 68.840176) (end 83.432824 65.532) (width 1) (layer "F.Cu") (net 4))
 (segment (start 64.262 77.724) (end 69.904 77.724) (width 1) (layer "F.Cu") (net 4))
 (segment (start 86.741 69.108) (end 86.741 68.840176) (width 1) (layer "F.Cu") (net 4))
 (segment (start 85.978 76.264) (end 85.852 76.39) (width 1) (layer "F.Cu") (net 3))
 (segment (start 64.262 69.724) (end 62.356 69.724) (width 1) (layer "F.Cu") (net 3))
 (segment (start 75.965 80.385) (end 75.965 71.235) (width 1) (layer "F.Cu") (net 3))
 (segment (start 66.168 69.724) (end 64.262 69.724) (width 1) (layer "F.Cu") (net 3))
 (segment (start 76.06 87.008) (end 75.438 87.63) (width 1) (layer "F.Cu") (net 3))
 (segment (start 87.884 76.264) (end 85.978 76.264) (width 1) (layer "F.Cu") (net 3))
 (segment (start 79.365 80.385) (end 79.365 74.635) (width 1) (layer "F.Cu") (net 3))
 (segment (start 76.915 89.154) (end 75.438 89.154) (width 1) (layer "F.Cu") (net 3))
 (segment (start 66.294 69.85) (end 66.168 69.724) (width 1) (layer "F.Cu") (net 3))
 (segment (start 90.5275 88.392) (end 89.154 88.392) (width 1) (layer "F.Cu") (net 3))
 (segment (start 87.884 76.264) (end 89.79 76.264) (width 1) (layer "F.Cu") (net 3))
 (segment (start 75.438 87.63) (end 75.438 89.154) (width 1) (layer "F.Cu") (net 3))
 (segment (start 62.356 69.724) (end 62.23 69.85) (width 1) (layer "F.Cu") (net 3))
 (segment (start 79.365 74.635) (end 75.965 71.235) (width 1) (layer "F.Cu") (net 3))
 (segment (start 89.79 76.264) (end 89.916 76.39) (width 1) (layer "F.Cu") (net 3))
 (segment (start 76.06 85.344) (end 76.06 87.008) (width 1) (layer "F.Cu") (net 3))
 (via (at 75.946 75.184) (size 1) (drill 0.6) (layers "F.Cu" "B.Cu") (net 3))
 (via (at 75.438 87.63) (size 1) (drill 0.6) (layers "F.Cu" "B.Cu") (free) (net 3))
 (via (at 89.154 88.392) (size 1) (drill 0.6) (layers "F.Cu" "B.Cu") (free) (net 3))
 (via (at 89.916 76.39) (size 1) (drill 0.6) (layers "F.Cu" "B.Cu") (free) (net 3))
 (via (at 71.374 75.184) (size 1) (drill 0.6) (layers "F.Cu" "B.Cu") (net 3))
 (via (at 75.438 89.154) (size 1) (drill 0.6) (layers "F.Cu" "B.Cu") (free) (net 3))
 (via (at 71.374 67.31) (size 1) (drill 0.6) (layers "F.Cu" "B.Cu") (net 3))
 (via (at 62.23 69.85) (size 1) (drill 0.6) (layers "F.Cu" "B.Cu") (free) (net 3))
 (via (at 85.852 76.39) (size 1) (drill 0.6) (layers "F.Cu" "B.Cu") (free) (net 3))
 (via (at 75.946 67.31) (size 1) (drill 0.6) (layers "F.Cu" "B.Cu") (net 3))
 (via (at 75.946 71.374) (size 1) (drill 0.6) (layers "F.Cu" "B.Cu") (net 3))
 (via (at 80.518 67.31) (size 1) (drill 0.6) (layers "F.Cu" "B.Cu") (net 3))
 (via (at 80.518 75.184) (size 1) (drill 0.6) (layers "F.Cu" "B.Cu") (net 3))
 (via (at 66.294 69.85) (size 1) (drill 0.6) (layers "F.Cu" "B.Cu") (free) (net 3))
 (via (at 71.374 71.374) (size 1) (drill 0.6) (layers "F.Cu" "B.Cu") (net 3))
 (via (at 80.518 71.374) (size 1) (drill 0.6) (layers "F.Cu" "B.Cu") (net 3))
 (segment (start 80.518 86.614) (end 80.772 86.868) (width 1) (layer "F.Cu") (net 2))
 (segment (start 64.262 90.51) (end 65.192 91.44) (width 1) (layer "F.Cu") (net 2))
 (segment (start 87.566 84.582) (end 87.884 84.264) (width 1) (layer "F.Cu") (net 2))
 (segment (start 93.726 78.422) (end 87.884 84.264) (width 1) (layer "F.Cu") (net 2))
 (segment (start 80.518 84.582) (end 80.518 86.614) (width 1) (layer "F.Cu") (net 2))
 (segment (start 65.192 91.44) (end 81.026 91.44) (width 1) (layer "F.Cu") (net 2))
 (segment (start 80.772 91.186) (end 81.026 91.44) (width 1) (layer "F.Cu") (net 2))
 (segment (start 80.772 86.868) (end 80.772 91.186) (width 1) (layer "F.Cu") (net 2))
 (segment (start 80.518 84.582) (end 87.566 84.582) (width 1) (layer "F.Cu") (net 2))
 (segment (start 93.726 69.108) (end 93.726 78.422) (width 1) (layer "F.Cu") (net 2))
 (segment (start 81.026 91.44) (end 90.5025 91.44) (width 1) (layer "F.Cu") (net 2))
 (segment (start 77.665 83.554) (end 78.693 84.582) (width 1) (layer "F.Cu") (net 5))
 (segment (start 78.693 89.107) (end 78.74 89.154) (width 1) (layer "F.Cu") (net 5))
 (segment (start 78.693 84.582) (end 78.693 89.107) (width 1) (layer "F.Cu") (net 5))
 (segment (start 77.665 80.385) (end 77.665 83.554) (width 1) (layer "F.Cu") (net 5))
 (segment (start 68.126 82.21) (end 64.262 82.21) (width 1) (layer "F.Cu") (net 1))
 (segment (start 74.265 83.215) (end 72.136 85.344) (width 1) (layer "F.Cu") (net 1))
 (segment (start 74.265 80.385) (end 74.265 83.215) (width 1) (layer "F.Cu") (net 1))
 (segment (start 71.26 85.344) (end 68.126 82.21) (width 1) (layer "F.Cu") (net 1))
 (segment (start 72.136 85.344) (end 71.26 85.344) (width 1) (layer "F.Cu") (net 1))
 (segment (start 92.3775 91.44) (end 92.3775 88.417) (width 1) (layer "F.Cu") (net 6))
 (segment (start 92.3775 88.417) (end 92.3525 88.392) (width 1) (layer "F.Cu") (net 6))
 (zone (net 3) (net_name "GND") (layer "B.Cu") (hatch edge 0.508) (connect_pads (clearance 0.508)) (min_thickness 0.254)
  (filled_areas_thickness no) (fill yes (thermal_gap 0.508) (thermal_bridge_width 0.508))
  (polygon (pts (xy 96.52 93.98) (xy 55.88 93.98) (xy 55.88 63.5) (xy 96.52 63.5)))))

